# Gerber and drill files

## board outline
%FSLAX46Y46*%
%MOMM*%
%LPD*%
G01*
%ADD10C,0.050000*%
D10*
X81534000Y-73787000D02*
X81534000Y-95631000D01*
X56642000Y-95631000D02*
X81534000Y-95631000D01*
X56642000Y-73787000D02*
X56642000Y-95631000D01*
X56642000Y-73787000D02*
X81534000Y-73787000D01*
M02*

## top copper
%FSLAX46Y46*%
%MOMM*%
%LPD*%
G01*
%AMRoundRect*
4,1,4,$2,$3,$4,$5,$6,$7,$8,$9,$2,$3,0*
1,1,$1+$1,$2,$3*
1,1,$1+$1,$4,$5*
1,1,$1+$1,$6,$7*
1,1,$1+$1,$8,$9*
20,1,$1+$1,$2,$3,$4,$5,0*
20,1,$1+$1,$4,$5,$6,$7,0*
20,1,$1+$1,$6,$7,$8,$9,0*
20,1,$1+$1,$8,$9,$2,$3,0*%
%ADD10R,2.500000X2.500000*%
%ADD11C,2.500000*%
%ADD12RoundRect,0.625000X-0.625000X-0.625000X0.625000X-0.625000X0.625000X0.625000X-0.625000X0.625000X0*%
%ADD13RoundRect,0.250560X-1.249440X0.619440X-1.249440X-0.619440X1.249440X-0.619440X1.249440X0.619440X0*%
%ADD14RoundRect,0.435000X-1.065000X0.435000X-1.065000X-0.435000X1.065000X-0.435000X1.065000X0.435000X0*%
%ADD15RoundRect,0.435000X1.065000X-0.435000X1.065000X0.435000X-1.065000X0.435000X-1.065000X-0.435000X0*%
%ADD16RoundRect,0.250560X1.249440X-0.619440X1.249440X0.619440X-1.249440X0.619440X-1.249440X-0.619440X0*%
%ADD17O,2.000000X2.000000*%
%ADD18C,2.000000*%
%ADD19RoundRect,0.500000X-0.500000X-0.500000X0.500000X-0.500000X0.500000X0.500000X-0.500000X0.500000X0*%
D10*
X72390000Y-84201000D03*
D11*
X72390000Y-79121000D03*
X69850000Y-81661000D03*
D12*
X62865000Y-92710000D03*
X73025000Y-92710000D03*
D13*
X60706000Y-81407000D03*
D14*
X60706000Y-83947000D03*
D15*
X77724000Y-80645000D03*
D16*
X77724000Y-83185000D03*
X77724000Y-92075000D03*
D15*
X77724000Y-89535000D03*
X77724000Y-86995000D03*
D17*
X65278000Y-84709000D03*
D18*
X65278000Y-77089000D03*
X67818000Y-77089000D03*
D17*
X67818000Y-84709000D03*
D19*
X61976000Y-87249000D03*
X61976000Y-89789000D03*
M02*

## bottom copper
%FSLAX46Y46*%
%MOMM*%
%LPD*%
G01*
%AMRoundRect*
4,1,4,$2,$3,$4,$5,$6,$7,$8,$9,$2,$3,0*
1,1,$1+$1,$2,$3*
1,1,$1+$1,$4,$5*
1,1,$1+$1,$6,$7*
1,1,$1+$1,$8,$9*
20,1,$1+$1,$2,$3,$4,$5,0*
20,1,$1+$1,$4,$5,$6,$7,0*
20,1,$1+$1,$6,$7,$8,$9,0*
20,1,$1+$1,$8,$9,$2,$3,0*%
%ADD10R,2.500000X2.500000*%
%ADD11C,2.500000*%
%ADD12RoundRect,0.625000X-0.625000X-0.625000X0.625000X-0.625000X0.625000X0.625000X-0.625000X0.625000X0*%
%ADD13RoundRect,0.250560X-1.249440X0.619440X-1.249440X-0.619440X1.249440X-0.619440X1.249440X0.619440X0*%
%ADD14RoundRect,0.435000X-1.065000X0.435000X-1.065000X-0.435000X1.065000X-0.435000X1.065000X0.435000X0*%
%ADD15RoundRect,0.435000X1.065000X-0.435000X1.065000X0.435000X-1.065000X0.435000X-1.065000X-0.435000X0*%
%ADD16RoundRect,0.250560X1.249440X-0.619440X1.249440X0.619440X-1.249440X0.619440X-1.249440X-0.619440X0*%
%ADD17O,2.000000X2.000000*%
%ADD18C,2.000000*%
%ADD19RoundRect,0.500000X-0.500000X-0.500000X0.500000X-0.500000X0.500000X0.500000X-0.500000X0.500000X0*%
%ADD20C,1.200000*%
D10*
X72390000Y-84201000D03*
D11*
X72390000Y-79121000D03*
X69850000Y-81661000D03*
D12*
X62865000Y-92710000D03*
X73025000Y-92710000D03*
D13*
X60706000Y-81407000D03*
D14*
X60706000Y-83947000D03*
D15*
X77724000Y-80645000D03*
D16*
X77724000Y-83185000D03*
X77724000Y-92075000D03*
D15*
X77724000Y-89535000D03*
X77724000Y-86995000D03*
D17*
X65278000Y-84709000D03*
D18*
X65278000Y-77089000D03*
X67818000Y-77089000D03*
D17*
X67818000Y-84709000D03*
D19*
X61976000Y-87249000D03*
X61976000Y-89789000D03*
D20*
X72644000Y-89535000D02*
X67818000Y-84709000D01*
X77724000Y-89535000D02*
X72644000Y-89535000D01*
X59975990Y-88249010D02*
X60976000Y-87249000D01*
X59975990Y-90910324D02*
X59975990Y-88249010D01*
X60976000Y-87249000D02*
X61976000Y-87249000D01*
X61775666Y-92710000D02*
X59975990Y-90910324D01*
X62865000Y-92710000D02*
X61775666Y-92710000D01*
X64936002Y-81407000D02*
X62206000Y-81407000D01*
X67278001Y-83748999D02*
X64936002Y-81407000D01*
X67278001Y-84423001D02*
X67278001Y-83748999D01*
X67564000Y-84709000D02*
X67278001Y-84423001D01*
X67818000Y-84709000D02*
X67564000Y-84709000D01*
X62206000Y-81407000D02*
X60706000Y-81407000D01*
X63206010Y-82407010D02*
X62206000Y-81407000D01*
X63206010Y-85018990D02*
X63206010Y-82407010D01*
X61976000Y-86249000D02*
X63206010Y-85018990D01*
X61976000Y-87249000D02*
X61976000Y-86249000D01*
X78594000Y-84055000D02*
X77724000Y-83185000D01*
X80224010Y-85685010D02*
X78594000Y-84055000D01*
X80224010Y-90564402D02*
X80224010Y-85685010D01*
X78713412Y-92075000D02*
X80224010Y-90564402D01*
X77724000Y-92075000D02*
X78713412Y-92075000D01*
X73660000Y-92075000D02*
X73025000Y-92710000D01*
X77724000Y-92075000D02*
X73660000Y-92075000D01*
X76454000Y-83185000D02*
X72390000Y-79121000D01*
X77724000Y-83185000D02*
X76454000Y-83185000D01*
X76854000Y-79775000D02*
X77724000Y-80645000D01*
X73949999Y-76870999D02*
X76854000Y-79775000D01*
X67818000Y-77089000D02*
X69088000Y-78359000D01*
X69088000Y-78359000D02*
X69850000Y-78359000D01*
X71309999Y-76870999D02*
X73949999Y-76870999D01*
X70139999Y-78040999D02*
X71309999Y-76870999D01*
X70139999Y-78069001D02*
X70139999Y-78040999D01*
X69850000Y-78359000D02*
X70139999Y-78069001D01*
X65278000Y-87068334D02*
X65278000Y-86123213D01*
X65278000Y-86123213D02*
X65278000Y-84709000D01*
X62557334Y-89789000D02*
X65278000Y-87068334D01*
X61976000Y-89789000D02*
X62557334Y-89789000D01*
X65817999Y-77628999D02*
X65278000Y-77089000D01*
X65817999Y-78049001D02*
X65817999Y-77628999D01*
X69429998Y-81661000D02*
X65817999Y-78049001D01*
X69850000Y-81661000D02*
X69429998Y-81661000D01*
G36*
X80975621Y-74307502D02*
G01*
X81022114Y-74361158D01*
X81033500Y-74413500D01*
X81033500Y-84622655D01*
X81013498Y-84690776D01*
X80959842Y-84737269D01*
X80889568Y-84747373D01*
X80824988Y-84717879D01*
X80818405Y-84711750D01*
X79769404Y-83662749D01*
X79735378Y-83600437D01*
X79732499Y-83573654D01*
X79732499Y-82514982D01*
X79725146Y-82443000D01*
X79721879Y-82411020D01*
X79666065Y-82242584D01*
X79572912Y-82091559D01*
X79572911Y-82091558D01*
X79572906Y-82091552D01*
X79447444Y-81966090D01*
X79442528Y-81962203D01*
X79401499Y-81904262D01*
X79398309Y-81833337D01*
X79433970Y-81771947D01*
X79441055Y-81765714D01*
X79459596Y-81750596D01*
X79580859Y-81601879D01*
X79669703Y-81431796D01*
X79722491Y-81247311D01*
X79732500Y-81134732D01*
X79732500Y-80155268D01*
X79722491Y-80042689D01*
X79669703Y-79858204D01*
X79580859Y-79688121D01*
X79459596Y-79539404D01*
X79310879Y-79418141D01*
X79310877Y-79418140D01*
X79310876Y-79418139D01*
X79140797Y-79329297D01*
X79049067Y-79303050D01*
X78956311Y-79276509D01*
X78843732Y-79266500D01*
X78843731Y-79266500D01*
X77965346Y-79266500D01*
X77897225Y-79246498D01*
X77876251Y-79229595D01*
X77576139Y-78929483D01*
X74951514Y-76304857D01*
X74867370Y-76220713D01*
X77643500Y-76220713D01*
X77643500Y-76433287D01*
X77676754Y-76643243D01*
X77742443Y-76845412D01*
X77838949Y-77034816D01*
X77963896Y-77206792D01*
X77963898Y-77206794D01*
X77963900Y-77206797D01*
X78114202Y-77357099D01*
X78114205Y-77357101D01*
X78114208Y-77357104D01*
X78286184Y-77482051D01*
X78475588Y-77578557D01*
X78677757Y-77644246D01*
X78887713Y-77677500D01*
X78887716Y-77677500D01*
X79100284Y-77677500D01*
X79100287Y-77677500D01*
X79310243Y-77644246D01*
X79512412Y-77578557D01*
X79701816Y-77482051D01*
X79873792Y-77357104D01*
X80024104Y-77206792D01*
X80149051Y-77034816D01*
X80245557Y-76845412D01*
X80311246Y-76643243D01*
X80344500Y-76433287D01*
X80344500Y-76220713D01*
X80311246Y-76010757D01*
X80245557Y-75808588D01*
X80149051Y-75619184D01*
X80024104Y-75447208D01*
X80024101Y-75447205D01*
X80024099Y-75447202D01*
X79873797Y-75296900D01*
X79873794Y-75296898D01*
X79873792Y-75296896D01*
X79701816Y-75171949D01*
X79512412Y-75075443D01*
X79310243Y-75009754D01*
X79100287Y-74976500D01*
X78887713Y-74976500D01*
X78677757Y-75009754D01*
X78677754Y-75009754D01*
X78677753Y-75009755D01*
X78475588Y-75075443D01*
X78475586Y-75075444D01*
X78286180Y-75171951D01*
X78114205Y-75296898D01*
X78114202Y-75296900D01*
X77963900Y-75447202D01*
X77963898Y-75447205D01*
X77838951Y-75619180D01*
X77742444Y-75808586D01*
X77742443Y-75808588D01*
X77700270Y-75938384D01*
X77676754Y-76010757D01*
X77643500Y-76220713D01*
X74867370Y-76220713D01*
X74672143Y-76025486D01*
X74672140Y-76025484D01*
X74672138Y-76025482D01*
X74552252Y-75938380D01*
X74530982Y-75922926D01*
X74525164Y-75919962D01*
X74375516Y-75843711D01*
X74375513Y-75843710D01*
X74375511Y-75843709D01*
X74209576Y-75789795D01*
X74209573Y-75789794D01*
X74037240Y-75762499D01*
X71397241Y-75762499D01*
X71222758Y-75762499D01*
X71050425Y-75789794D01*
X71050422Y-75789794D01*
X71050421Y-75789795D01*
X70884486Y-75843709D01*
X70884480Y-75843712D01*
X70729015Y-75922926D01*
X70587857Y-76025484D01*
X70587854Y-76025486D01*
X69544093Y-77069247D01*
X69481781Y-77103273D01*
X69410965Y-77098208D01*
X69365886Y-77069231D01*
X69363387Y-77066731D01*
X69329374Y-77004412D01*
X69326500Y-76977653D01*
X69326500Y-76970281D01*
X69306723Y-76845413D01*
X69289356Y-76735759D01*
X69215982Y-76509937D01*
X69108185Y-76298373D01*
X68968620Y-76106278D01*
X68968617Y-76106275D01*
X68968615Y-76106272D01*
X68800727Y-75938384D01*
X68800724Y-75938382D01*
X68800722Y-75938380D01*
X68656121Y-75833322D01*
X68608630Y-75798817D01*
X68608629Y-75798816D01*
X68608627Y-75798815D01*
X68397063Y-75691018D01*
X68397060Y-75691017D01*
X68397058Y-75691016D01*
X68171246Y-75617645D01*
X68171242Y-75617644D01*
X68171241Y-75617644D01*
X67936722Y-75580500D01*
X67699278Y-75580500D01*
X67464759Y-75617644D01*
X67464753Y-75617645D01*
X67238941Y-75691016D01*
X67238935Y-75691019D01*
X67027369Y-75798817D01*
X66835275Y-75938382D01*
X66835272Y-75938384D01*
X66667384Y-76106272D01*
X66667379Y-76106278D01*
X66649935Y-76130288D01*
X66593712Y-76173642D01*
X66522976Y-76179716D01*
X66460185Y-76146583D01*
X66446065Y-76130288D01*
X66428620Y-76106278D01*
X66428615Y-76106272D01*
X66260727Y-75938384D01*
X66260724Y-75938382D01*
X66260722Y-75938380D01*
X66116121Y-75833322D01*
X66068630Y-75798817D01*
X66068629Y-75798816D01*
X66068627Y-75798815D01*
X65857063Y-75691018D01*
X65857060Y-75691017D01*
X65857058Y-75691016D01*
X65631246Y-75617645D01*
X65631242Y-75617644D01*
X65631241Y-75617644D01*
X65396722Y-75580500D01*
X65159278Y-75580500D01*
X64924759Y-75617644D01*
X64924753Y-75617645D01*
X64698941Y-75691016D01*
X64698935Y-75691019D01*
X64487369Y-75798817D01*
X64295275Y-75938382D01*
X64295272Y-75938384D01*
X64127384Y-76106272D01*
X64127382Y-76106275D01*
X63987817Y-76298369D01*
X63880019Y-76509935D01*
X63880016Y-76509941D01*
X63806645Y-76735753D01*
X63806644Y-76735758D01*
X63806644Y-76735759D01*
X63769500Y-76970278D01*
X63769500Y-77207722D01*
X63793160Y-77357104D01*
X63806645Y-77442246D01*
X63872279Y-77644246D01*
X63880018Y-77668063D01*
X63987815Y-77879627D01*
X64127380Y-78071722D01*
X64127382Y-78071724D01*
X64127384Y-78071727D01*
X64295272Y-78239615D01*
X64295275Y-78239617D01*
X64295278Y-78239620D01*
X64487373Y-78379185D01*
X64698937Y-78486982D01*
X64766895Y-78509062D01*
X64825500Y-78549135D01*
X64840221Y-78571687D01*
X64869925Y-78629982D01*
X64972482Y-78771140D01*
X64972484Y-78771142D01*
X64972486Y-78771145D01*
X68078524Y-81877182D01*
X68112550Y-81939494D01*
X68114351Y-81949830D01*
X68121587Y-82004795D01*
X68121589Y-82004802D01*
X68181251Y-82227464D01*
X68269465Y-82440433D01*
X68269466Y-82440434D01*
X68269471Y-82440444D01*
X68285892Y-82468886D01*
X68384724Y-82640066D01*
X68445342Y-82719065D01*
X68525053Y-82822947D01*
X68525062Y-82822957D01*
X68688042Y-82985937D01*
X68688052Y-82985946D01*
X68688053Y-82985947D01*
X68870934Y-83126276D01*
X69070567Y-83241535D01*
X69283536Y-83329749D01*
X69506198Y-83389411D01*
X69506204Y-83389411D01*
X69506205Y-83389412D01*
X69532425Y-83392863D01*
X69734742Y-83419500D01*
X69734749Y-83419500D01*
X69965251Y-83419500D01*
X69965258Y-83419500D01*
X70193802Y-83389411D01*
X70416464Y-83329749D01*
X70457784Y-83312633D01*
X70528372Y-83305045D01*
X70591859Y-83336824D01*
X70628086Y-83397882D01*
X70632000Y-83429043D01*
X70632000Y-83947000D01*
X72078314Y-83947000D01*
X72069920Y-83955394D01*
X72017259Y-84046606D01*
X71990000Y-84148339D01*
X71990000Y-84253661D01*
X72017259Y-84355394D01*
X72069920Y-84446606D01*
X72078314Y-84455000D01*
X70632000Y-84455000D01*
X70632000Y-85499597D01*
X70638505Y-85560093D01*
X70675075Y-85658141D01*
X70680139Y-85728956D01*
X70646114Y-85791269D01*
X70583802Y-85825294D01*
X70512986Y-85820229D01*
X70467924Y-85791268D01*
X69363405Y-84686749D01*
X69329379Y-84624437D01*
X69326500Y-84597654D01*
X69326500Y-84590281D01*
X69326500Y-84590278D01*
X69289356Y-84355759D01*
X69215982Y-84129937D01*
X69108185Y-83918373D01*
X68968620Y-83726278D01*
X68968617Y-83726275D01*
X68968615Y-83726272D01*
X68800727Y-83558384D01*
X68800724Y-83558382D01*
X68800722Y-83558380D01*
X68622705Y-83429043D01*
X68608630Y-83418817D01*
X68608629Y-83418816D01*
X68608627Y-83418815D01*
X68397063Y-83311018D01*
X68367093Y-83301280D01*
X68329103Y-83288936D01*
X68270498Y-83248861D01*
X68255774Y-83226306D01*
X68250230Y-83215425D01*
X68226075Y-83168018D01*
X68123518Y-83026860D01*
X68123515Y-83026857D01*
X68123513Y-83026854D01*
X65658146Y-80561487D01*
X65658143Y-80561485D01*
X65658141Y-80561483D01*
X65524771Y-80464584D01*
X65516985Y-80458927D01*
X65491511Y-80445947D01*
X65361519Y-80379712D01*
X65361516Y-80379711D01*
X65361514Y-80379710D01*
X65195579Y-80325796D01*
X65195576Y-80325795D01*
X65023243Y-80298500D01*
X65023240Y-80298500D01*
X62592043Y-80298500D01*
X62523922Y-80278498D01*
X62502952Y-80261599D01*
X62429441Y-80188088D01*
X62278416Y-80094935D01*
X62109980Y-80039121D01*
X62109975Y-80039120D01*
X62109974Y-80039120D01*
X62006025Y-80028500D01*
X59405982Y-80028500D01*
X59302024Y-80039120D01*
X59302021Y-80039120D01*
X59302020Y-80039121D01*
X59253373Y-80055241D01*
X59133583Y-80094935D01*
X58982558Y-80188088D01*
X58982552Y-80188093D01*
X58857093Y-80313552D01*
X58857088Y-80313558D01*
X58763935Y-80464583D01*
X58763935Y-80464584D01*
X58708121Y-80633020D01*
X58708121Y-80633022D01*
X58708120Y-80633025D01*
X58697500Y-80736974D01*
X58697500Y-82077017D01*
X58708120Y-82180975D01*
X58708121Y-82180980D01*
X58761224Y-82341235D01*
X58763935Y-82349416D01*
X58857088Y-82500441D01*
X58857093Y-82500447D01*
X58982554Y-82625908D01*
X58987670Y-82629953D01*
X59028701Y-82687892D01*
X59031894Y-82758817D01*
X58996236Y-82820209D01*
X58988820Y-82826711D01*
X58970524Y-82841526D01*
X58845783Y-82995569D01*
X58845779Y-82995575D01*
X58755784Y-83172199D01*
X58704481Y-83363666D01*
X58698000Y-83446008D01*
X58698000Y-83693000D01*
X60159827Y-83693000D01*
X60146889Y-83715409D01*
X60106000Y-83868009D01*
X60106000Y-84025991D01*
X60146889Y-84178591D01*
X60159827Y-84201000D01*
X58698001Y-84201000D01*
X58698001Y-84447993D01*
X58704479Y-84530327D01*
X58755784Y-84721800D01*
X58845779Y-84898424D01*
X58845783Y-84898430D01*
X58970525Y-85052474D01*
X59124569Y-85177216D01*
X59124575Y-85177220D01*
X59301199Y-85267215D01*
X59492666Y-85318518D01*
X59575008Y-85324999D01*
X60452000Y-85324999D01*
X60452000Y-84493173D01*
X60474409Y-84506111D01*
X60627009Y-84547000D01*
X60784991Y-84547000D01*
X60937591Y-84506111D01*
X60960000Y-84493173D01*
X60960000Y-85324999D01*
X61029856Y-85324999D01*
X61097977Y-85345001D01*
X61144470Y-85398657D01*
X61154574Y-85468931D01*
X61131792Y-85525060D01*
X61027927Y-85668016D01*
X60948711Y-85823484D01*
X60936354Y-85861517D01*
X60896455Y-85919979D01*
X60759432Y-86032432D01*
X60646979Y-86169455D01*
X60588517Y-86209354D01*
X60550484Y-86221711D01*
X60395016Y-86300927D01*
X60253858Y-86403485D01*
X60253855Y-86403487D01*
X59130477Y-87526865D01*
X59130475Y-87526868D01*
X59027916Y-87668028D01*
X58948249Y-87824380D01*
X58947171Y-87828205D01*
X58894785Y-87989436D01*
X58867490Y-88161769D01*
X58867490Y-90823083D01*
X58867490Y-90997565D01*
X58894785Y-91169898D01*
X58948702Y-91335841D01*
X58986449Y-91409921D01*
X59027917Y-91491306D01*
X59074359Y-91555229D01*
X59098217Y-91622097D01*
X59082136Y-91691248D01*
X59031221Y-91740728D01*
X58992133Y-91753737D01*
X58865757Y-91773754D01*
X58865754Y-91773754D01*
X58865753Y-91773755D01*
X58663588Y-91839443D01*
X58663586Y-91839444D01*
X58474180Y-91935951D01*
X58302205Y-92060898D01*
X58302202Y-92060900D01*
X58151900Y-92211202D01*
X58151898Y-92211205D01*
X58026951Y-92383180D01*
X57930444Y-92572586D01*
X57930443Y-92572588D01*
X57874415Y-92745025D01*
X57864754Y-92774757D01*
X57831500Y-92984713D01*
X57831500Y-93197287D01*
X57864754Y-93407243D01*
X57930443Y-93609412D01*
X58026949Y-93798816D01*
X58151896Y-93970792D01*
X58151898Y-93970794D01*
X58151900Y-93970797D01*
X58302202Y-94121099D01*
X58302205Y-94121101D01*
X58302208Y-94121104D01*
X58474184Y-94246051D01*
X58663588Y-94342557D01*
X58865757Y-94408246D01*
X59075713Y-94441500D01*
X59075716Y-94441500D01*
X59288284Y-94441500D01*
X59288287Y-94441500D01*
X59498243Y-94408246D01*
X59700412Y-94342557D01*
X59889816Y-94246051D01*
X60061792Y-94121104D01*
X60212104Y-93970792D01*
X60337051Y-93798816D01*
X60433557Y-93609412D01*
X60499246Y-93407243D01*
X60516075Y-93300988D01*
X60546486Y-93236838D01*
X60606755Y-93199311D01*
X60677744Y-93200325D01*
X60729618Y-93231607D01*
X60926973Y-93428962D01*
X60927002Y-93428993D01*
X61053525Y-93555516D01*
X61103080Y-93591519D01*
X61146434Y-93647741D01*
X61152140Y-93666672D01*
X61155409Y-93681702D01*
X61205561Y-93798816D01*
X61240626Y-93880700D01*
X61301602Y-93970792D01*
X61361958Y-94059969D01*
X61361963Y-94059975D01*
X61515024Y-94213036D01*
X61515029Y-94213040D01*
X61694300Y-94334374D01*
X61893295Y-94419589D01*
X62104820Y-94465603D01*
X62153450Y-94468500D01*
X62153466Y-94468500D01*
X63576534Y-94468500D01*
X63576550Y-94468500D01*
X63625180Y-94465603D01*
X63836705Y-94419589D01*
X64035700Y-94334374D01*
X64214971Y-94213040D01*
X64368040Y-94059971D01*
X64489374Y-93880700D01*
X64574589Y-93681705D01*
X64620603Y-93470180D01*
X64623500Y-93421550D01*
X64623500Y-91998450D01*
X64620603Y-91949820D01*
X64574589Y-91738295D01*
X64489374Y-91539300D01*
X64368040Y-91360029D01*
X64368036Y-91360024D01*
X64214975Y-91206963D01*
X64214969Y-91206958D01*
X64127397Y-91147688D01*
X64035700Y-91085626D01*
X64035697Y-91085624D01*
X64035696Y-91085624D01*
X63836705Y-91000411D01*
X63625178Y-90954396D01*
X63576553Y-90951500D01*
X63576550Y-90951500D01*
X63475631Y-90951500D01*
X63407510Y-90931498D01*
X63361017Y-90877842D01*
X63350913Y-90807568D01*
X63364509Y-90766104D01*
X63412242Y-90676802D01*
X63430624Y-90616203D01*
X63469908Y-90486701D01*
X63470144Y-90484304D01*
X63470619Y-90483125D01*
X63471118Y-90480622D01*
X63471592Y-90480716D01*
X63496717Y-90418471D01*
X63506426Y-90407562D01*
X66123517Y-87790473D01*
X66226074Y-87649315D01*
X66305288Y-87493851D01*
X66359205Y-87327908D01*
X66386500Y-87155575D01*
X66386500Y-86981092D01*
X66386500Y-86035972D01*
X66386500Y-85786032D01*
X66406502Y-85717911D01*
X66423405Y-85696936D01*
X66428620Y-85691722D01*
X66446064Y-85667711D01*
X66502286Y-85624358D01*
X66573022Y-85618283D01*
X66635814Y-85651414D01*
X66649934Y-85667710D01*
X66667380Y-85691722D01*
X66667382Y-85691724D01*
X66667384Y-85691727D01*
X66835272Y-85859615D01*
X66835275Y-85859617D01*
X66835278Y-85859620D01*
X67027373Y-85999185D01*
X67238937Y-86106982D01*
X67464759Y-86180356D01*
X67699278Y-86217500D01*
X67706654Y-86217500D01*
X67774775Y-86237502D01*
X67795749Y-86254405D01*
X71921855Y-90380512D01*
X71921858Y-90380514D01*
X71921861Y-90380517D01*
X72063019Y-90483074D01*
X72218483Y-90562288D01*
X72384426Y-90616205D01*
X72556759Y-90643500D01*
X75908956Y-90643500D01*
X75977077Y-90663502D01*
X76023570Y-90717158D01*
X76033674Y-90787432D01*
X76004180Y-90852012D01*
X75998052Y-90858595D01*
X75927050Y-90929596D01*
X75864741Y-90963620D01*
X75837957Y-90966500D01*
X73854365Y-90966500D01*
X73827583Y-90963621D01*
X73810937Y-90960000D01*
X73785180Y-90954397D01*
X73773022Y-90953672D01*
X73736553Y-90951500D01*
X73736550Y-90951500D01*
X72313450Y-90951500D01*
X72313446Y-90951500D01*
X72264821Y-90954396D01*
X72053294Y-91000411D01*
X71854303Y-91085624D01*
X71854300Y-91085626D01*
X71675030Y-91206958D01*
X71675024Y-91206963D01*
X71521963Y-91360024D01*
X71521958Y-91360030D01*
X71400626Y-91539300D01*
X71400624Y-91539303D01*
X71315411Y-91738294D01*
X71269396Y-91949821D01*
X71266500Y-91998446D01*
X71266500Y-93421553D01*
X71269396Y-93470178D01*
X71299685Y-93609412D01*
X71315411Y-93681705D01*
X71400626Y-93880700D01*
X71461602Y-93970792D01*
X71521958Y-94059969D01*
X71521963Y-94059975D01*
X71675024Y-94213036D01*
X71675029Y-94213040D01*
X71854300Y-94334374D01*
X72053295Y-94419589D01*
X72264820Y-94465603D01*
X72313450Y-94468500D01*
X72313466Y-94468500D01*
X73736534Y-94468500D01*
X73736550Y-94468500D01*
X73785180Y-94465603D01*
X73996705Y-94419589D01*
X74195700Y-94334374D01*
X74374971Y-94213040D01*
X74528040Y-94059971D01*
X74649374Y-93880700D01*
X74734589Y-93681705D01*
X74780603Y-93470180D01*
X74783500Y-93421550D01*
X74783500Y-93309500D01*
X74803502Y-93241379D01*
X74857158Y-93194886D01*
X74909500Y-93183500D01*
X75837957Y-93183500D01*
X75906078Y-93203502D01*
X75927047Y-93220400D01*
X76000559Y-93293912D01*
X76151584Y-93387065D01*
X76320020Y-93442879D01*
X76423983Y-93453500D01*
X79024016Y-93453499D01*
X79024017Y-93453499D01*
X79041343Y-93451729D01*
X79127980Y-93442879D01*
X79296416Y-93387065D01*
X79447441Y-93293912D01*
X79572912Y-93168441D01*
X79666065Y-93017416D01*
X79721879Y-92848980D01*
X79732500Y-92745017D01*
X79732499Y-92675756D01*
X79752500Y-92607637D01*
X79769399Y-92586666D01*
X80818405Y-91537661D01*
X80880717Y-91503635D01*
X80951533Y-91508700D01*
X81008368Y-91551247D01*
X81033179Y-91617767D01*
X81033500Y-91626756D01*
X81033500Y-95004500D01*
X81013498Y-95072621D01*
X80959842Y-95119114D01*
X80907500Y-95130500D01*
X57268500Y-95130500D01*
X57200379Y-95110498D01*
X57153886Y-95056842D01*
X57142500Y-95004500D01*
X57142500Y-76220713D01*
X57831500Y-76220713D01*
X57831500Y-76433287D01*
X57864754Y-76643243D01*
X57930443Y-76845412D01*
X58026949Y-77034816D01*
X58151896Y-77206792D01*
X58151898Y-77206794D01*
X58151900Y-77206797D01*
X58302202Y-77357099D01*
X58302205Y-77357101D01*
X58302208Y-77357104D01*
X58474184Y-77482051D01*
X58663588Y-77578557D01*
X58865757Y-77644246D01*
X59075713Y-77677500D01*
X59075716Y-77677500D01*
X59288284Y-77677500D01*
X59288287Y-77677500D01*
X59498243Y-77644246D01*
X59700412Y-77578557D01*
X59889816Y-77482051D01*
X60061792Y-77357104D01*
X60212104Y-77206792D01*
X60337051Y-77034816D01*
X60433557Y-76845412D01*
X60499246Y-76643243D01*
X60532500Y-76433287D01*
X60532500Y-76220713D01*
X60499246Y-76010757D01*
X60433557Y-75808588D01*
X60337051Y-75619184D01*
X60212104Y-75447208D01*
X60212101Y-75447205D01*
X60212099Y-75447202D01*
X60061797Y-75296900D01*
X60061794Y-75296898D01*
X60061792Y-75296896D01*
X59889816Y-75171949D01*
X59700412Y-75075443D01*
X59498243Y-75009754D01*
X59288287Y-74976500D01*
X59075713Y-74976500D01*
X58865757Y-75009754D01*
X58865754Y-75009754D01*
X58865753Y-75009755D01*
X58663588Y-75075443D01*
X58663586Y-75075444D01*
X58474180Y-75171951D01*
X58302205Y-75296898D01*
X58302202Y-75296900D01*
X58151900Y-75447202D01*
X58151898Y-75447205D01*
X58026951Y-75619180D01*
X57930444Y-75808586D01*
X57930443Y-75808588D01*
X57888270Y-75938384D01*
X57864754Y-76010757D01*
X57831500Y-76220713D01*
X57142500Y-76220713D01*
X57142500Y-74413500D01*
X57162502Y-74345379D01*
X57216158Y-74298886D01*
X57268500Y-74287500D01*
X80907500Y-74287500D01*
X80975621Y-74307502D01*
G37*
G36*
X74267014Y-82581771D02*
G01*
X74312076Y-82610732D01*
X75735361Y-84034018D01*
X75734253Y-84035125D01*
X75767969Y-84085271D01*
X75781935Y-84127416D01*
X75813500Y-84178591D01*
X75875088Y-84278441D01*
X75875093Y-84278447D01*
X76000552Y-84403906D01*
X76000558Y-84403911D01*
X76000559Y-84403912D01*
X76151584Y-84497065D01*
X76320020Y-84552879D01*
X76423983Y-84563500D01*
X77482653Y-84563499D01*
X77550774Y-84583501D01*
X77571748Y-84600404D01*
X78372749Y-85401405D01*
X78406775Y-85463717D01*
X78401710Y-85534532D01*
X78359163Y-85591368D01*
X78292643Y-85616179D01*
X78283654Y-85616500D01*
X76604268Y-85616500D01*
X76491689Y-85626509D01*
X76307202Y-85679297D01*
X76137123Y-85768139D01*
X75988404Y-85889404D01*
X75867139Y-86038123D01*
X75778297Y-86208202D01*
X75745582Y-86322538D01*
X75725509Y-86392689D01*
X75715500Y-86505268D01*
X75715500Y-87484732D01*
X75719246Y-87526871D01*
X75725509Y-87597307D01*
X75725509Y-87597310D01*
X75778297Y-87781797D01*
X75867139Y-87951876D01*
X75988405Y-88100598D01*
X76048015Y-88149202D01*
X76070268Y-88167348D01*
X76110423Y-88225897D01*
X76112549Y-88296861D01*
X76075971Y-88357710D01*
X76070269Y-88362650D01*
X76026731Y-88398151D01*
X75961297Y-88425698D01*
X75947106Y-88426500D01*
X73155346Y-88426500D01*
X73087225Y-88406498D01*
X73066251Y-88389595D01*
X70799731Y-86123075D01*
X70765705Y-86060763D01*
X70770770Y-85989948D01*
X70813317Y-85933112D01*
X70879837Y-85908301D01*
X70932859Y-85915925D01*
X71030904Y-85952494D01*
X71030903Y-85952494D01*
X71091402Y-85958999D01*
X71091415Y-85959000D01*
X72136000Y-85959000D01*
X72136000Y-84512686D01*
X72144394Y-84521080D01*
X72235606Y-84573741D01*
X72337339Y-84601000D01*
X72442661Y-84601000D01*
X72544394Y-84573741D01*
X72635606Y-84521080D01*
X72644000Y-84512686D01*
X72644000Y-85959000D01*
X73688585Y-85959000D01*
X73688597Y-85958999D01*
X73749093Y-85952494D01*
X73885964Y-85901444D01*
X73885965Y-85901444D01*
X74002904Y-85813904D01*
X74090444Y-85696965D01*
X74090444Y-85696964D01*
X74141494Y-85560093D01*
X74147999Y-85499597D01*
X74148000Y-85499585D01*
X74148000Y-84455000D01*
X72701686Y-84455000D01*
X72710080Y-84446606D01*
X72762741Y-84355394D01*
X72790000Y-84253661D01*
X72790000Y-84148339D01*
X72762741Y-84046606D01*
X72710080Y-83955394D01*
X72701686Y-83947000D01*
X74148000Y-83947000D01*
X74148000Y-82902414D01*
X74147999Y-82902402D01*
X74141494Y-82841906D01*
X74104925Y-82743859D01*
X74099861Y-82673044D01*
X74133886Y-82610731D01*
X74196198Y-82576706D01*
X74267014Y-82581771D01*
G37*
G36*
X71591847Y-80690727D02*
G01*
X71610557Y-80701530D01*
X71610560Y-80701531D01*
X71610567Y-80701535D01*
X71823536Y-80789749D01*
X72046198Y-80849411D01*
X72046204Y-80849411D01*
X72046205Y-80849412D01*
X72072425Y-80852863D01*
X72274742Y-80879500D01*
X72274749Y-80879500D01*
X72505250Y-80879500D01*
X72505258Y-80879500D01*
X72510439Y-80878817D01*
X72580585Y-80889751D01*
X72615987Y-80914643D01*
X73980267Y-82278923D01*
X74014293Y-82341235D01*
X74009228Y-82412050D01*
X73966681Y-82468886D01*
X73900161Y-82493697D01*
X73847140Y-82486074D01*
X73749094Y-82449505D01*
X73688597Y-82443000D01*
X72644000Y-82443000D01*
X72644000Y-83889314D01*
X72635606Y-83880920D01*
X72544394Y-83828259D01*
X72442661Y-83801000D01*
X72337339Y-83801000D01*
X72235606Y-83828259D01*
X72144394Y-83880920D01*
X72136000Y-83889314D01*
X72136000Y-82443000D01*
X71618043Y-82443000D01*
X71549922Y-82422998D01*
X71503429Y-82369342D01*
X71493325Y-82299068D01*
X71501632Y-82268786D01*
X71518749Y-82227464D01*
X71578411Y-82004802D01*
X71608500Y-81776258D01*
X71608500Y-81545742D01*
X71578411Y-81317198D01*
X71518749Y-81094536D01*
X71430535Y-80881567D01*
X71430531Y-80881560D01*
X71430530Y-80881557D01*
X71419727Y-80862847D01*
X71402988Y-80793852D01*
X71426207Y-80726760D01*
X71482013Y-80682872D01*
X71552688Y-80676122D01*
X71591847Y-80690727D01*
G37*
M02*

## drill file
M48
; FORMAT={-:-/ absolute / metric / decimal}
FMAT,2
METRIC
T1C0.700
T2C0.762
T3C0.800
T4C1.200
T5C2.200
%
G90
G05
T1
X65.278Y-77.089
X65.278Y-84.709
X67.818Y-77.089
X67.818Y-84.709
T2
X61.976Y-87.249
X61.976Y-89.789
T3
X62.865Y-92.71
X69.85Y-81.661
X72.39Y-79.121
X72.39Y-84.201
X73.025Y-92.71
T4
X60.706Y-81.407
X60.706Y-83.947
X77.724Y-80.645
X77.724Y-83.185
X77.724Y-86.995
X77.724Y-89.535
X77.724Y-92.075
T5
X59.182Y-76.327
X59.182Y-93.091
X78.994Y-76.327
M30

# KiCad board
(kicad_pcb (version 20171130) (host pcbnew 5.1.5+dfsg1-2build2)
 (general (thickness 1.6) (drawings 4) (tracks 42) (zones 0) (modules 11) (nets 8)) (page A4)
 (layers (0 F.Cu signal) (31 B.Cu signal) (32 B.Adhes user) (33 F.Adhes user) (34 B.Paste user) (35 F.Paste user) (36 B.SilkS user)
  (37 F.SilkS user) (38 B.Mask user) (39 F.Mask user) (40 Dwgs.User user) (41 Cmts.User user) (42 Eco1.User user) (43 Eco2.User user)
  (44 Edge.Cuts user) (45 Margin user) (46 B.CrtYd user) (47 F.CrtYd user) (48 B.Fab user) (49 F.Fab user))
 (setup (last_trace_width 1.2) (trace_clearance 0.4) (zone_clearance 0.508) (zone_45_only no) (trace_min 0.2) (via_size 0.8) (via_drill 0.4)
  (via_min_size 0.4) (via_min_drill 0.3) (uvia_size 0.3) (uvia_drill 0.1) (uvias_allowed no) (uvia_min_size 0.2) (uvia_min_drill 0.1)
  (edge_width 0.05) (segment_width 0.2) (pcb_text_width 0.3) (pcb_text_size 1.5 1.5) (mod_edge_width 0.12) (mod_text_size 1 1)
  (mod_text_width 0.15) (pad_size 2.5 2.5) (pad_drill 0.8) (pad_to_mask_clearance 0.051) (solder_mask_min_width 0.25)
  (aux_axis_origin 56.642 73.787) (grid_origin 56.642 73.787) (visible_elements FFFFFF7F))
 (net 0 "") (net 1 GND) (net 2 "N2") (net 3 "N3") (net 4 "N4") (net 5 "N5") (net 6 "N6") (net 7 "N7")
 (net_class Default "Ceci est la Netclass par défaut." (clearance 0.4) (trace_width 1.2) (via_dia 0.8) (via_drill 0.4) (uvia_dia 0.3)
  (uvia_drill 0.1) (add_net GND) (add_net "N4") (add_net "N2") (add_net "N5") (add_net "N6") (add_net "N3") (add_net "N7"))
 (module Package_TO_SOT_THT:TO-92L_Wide (layer F.Cu) (at 72.39 84.201 90)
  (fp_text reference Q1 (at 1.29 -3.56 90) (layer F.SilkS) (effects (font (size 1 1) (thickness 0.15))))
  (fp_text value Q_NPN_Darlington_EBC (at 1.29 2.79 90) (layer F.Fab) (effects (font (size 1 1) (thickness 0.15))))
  (pad 1 thru_hole rect (at 0 0 180) (size 2.5 2.5) (drill 0.8) (layers *.Cu *.Mask) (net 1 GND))
  (pad 3 thru_hole circle (at 5.08 0 180) (size 2.5 2.5) (drill 0.8) (layers *.Cu *.Mask) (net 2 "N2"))
  (pad 2 thru_hole circle (at 2.54 -2.54 180) (size 2.5 2.5) (drill 0.8) (layers *.Cu *.Mask) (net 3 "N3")))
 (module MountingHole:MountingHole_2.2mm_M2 (layer F.Cu) (at 78.994 76.327)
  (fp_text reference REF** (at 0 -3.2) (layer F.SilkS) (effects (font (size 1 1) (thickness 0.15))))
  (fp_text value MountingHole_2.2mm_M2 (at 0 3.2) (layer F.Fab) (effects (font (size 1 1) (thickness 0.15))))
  (pad 1 np_thru_hole circle (at 0 0) (size 2.2 2.2) (drill 2.2) (layers *.Cu *.Mask)))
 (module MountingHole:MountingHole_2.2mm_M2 (layer F.Cu) (at 59.182 93.091)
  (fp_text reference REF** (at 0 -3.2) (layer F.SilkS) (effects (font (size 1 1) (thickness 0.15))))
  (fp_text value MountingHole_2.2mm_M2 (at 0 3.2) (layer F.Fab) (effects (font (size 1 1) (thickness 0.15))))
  (pad 1 np_thru_hole circle (at 0 0) (size 2.2 2.2) (drill 2.2) (layers *.Cu *.Mask)))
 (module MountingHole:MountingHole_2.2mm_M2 (layer F.Cu) (at 59.182 76.327)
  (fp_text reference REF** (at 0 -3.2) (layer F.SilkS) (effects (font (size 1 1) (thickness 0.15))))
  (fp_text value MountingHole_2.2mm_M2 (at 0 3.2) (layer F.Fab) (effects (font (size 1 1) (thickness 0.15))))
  (pad 1 np_thru_hole circle (at 0 0) (size 2.2 2.2) (drill 2.2) (layers *.Cu *.Mask)))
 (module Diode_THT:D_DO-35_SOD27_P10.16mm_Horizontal (layer F.Cu) (at 62.865 92.71)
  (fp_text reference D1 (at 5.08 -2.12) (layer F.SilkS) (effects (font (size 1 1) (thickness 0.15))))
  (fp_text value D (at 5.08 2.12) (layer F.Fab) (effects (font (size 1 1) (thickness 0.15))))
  (pad 1 thru_hole roundrect (at 0 0) (size 2.5 2.5) (drill 0.8) (layers *.Cu *.Mask) (roundrect_rratio 0.25) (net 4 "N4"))
  (pad 2 thru_hole roundrect (at 10.16 0) (size 2.5 2.5) (drill 0.8) (layers *.Cu *.Mask) (roundrect_rratio 0.25) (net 2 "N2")))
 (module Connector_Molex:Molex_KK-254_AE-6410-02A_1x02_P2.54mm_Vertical (layer F.Cu) (at 60.706 81.407 270)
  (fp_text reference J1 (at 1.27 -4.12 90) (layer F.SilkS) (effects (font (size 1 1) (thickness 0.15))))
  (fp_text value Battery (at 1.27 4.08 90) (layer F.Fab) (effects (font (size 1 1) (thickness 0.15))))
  (pad 1 thru_hole roundrect (at 0 0 270) (size 1.74 3) (drill 1.2) (layers *.Cu *.Mask) (roundrect_rratio 0.144) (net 4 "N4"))
  (pad 2 thru_hole roundrect (at 2.54 0 270) (size 1.74 3) (drill 1.2) (layers *.Cu *.Mask) (roundrect_rratio 0.25) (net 1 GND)))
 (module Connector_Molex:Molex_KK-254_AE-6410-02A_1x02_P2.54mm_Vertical (layer F.Cu) (at 77.724 83.185 90)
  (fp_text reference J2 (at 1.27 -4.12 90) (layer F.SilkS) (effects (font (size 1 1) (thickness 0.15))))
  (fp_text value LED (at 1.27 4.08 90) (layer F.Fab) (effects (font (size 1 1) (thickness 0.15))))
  (pad 2 thru_hole roundrect (at 2.54 0 90) (size 1.74 3) (drill 1.2) (layers *.Cu *.Mask) (roundrect_rratio 0.25) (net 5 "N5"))
  (pad 1 thru_hole roundrect (at 0 0 90) (size 1.74 3) (drill 1.2) (layers *.Cu *.Mask) (roundrect_rratio 0.144) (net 2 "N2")))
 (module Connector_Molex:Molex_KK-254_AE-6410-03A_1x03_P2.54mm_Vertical (layer F.Cu) (at 77.724 92.075 90)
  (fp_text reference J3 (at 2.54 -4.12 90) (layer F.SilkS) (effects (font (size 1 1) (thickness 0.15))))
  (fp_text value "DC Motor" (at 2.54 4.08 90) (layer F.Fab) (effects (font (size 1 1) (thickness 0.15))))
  (pad 1 thru_hole roundrect (at 0 0 90) (size 1.74 3) (drill 1.2) (layers *.Cu *.Mask) (roundrect_rratio 0.144) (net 2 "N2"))
  (pad 2 thru_hole roundrect (at 2.54 0 90) (size 1.74 3) (drill 1.2) (layers *.Cu *.Mask) (roundrect_rratio 0.25) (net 4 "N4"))
  (pad 3 thru_hole roundrect (at 5.08 0 90) (size 1.74 3) (drill 1.2) (layers *.Cu *.Mask) (roundrect_rratio 0.25) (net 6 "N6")))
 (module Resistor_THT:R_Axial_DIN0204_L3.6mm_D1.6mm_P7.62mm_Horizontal (layer F.Cu) (at 65.278 77.089 270)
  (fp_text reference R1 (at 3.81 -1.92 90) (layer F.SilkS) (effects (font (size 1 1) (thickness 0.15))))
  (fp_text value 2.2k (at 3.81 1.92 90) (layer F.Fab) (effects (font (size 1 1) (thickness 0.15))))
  (pad 2 thru_hole oval (at 7.62 0 270) (size 2 2) (drill 0.7) (layers *.Cu *.Mask) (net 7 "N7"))
  (pad 1 thru_hole circle (at 0 0 270) (size 2 2) (drill 0.7) (layers *.Cu *.Mask) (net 3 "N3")))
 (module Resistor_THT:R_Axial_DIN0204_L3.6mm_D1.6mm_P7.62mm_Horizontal (layer F.Cu) (at 67.818 77.089 270)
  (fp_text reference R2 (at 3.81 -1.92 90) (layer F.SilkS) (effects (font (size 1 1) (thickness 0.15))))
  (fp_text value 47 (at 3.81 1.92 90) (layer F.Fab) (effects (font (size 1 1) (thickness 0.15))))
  (pad 1 thru_hole circle (at 0 0 270) (size 2 2) (drill 0.7) (layers *.Cu *.Mask) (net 5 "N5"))
  (pad 2 thru_hole oval (at 7.62 0 270) (size 2 2) (drill 0.7) (layers *.Cu *.Mask) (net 4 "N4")))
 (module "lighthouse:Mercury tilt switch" (layer F.Cu) (at 61.976 87.249)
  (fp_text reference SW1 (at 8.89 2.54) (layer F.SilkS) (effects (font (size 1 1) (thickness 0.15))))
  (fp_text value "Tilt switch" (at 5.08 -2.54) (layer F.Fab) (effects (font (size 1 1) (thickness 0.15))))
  (pad 1 thru_hole roundrect (at 0 0) (size 2 2) (drill 0.762) (layers *.Cu *.Mask) (roundrect_rratio 0.25) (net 4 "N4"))
  (pad 2 thru_hole roundrect (at 0 2.54) (size 2 2) (drill 0.762) (layers *.Cu *.Mask) (roundrect_rratio 0.25) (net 7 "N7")))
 (gr_line (start 81.534 73.787) (end 81.534 95.631) (layer Edge.Cuts) (width 0.05))
 (gr_line (start 56.642 95.631) (end 81.534 95.631) (layer Edge.Cuts) (width 0.05))
 (gr_line (start 56.642 73.787) (end 56.642 95.631) (layer Edge.Cuts) (width 0.05))
 (gr_line (start 56.642 73.787) (end 81.534 73.787) (layer Edge.Cuts) (width 0.05))
 (segment (start 72.644 89.535) (end 67.818 84.709) (width 1.2) (layer B.Cu) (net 4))
 (segment (start 77.724 89.535) (end 72.644 89.535) (width 1.2) (layer B.Cu) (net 4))
 (segment (start 59.97599 88.24901) (end 60.976 87.249) (width 1.2) (layer B.Cu) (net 4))
 (segment (start 59.97599 90.910324) (end 59.97599 88.24901) (width 1.2) (layer B.Cu) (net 4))
 (segment (start 60.976 87.249) (end 61.976 87.249) (width 1.2) (layer B.Cu) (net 4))
 (segment (start 61.775666 92.71) (end 59.97599 90.910324) (width 1.2) (layer B.Cu) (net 4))
 (segment (start 62.865 92.71) (end 61.775666 92.71) (width 1.2) (layer B.Cu) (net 4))
 (segment (start 64.936002 81.407) (end 62.206 81.407) (width 1.2) (layer B.Cu) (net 4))
 (segment (start 67.278001 83.748999) (end 64.936002 81.407) (width 1.2) (layer B.Cu) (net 4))
 (segment (start 67.278001 84.423001) (end 67.278001 83.748999) (width 1.2) (layer B.Cu) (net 4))
 (segment (start 67.564 84.709) (end 67.278001 84.423001) (width 1.2) (layer B.Cu) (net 4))
 (segment (start 67.818 84.709) (end 67.564 84.709) (width 1.2) (layer B.Cu) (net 4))
 (segment (start 62.206 81.407) (end 60.706 81.407) (width 1.2) (layer B.Cu) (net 4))
 (segment (start 63.20601 82.40701) (end 62.206 81.407) (width 1.2) (layer B.Cu) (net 4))
 (segment (start 63.20601 85.01899) (end 63.20601 82.40701) (width 1.2) (layer B.Cu) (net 4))
 (segment (start 61.976 86.249) (end 63.20601 85.01899) (width 1.2) (layer B.Cu) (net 4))
 (segment (start 61.976 87.249) (end 61.976 86.249) (width 1.2) (layer B.Cu) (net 4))
 (segment (start 78.594 84.055) (end 77.724 83.185) (width 1.2) (layer B.Cu) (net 2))
 (segment (start 80.22401 85.68501) (end 78.594 84.055) (width 1.2) (layer B.Cu) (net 2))
 (segment (start 80.22401 90.564402) (end 80.22401 85.68501) (width 1.2) (layer B.Cu) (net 2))
 (segment (start 78.713412 92.075) (end 80.22401 90.564402) (width 1.2) (layer B.Cu) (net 2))
 (segment (start 77.724 92.075) (end 78.713412 92.075) (width 1.2) (layer B.Cu) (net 2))
 (segment (start 73.66 92.075) (end 73.025 92.71) (width 1.2) (layer B.Cu) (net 2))
 (segment (start 77.724 92.075) (end 73.66 92.075) (width 1.2) (layer B.Cu) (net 2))
 (segment (start 76.454 83.185) (end 72.39 79.121) (width 1.2) (layer B.Cu) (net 2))
 (segment (start 77.724 83.185) (end 76.454 83.185) (width 1.2) (layer B.Cu) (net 2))
 (segment (start 76.854 79.775) (end 77.724 80.645) (width 1.2) (layer B.Cu) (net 5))
 (segment (start 73.949999 76.870999) (end 76.854 79.775) (width 1.2) (layer B.Cu) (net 5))
 (segment (start 67.818 77.089) (end 69.088 78.359) (width 1.2) (layer B.Cu) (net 5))
 (segment (start 69.088 78.359) (end 69.85 78.359) (width 1.2) (layer B.Cu) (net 5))
 (segment (start 71.309999 76.870999) (end 73.949999 76.870999) (width 1.2) (layer B.Cu) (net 5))
 (segment (start 70.139999 78.040999) (end 71.309999 76.870999) (width 1.2) (layer B.Cu) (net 5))
 (segment (start 70.139999 78.069001) (end 70.139999 78.040999) (width 1.2) (layer B.Cu) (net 5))
 (segment (start 69.85 78.359) (end 70.139999 78.069001) (width 1.2) (layer B.Cu) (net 5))
 (segment (start 65.278 87.068334) (end 65.278 86.123213) (width 1.2) (layer B.Cu) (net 7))
 (segment (start 65.278 86.123213) (end 65.278 84.709) (width 1.2) (layer B.Cu) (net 7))
 (segment (start 62.557334 89.789) (end 65.278 87.068334) (width 1.2) (layer B.Cu) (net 7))
 (segment (start 61.976 89.789) (end 62.557334 89.789) (width 1.2) (layer B.Cu) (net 7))
 (segment (start 65.817999 77.628999) (end 65.278 77.089) (width 1.2) (layer B.Cu) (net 3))
 (segment (start 65.817999 78.049001) (end 65.817999 77.628999) (width 1.2) (layer B.Cu) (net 3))
 (segment (start 69.429998 81.661) (end 65.817999 78.049001) (width 1.2) (layer B.Cu) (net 3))
 (segment (start 69.85 81.661) (end 69.429998 81.661) (width 1.2) (layer B.Cu) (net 3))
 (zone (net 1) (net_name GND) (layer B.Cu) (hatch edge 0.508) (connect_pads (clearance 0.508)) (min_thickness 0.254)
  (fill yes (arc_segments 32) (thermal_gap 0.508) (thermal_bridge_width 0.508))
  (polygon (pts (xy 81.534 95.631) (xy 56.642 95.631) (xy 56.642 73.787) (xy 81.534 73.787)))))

